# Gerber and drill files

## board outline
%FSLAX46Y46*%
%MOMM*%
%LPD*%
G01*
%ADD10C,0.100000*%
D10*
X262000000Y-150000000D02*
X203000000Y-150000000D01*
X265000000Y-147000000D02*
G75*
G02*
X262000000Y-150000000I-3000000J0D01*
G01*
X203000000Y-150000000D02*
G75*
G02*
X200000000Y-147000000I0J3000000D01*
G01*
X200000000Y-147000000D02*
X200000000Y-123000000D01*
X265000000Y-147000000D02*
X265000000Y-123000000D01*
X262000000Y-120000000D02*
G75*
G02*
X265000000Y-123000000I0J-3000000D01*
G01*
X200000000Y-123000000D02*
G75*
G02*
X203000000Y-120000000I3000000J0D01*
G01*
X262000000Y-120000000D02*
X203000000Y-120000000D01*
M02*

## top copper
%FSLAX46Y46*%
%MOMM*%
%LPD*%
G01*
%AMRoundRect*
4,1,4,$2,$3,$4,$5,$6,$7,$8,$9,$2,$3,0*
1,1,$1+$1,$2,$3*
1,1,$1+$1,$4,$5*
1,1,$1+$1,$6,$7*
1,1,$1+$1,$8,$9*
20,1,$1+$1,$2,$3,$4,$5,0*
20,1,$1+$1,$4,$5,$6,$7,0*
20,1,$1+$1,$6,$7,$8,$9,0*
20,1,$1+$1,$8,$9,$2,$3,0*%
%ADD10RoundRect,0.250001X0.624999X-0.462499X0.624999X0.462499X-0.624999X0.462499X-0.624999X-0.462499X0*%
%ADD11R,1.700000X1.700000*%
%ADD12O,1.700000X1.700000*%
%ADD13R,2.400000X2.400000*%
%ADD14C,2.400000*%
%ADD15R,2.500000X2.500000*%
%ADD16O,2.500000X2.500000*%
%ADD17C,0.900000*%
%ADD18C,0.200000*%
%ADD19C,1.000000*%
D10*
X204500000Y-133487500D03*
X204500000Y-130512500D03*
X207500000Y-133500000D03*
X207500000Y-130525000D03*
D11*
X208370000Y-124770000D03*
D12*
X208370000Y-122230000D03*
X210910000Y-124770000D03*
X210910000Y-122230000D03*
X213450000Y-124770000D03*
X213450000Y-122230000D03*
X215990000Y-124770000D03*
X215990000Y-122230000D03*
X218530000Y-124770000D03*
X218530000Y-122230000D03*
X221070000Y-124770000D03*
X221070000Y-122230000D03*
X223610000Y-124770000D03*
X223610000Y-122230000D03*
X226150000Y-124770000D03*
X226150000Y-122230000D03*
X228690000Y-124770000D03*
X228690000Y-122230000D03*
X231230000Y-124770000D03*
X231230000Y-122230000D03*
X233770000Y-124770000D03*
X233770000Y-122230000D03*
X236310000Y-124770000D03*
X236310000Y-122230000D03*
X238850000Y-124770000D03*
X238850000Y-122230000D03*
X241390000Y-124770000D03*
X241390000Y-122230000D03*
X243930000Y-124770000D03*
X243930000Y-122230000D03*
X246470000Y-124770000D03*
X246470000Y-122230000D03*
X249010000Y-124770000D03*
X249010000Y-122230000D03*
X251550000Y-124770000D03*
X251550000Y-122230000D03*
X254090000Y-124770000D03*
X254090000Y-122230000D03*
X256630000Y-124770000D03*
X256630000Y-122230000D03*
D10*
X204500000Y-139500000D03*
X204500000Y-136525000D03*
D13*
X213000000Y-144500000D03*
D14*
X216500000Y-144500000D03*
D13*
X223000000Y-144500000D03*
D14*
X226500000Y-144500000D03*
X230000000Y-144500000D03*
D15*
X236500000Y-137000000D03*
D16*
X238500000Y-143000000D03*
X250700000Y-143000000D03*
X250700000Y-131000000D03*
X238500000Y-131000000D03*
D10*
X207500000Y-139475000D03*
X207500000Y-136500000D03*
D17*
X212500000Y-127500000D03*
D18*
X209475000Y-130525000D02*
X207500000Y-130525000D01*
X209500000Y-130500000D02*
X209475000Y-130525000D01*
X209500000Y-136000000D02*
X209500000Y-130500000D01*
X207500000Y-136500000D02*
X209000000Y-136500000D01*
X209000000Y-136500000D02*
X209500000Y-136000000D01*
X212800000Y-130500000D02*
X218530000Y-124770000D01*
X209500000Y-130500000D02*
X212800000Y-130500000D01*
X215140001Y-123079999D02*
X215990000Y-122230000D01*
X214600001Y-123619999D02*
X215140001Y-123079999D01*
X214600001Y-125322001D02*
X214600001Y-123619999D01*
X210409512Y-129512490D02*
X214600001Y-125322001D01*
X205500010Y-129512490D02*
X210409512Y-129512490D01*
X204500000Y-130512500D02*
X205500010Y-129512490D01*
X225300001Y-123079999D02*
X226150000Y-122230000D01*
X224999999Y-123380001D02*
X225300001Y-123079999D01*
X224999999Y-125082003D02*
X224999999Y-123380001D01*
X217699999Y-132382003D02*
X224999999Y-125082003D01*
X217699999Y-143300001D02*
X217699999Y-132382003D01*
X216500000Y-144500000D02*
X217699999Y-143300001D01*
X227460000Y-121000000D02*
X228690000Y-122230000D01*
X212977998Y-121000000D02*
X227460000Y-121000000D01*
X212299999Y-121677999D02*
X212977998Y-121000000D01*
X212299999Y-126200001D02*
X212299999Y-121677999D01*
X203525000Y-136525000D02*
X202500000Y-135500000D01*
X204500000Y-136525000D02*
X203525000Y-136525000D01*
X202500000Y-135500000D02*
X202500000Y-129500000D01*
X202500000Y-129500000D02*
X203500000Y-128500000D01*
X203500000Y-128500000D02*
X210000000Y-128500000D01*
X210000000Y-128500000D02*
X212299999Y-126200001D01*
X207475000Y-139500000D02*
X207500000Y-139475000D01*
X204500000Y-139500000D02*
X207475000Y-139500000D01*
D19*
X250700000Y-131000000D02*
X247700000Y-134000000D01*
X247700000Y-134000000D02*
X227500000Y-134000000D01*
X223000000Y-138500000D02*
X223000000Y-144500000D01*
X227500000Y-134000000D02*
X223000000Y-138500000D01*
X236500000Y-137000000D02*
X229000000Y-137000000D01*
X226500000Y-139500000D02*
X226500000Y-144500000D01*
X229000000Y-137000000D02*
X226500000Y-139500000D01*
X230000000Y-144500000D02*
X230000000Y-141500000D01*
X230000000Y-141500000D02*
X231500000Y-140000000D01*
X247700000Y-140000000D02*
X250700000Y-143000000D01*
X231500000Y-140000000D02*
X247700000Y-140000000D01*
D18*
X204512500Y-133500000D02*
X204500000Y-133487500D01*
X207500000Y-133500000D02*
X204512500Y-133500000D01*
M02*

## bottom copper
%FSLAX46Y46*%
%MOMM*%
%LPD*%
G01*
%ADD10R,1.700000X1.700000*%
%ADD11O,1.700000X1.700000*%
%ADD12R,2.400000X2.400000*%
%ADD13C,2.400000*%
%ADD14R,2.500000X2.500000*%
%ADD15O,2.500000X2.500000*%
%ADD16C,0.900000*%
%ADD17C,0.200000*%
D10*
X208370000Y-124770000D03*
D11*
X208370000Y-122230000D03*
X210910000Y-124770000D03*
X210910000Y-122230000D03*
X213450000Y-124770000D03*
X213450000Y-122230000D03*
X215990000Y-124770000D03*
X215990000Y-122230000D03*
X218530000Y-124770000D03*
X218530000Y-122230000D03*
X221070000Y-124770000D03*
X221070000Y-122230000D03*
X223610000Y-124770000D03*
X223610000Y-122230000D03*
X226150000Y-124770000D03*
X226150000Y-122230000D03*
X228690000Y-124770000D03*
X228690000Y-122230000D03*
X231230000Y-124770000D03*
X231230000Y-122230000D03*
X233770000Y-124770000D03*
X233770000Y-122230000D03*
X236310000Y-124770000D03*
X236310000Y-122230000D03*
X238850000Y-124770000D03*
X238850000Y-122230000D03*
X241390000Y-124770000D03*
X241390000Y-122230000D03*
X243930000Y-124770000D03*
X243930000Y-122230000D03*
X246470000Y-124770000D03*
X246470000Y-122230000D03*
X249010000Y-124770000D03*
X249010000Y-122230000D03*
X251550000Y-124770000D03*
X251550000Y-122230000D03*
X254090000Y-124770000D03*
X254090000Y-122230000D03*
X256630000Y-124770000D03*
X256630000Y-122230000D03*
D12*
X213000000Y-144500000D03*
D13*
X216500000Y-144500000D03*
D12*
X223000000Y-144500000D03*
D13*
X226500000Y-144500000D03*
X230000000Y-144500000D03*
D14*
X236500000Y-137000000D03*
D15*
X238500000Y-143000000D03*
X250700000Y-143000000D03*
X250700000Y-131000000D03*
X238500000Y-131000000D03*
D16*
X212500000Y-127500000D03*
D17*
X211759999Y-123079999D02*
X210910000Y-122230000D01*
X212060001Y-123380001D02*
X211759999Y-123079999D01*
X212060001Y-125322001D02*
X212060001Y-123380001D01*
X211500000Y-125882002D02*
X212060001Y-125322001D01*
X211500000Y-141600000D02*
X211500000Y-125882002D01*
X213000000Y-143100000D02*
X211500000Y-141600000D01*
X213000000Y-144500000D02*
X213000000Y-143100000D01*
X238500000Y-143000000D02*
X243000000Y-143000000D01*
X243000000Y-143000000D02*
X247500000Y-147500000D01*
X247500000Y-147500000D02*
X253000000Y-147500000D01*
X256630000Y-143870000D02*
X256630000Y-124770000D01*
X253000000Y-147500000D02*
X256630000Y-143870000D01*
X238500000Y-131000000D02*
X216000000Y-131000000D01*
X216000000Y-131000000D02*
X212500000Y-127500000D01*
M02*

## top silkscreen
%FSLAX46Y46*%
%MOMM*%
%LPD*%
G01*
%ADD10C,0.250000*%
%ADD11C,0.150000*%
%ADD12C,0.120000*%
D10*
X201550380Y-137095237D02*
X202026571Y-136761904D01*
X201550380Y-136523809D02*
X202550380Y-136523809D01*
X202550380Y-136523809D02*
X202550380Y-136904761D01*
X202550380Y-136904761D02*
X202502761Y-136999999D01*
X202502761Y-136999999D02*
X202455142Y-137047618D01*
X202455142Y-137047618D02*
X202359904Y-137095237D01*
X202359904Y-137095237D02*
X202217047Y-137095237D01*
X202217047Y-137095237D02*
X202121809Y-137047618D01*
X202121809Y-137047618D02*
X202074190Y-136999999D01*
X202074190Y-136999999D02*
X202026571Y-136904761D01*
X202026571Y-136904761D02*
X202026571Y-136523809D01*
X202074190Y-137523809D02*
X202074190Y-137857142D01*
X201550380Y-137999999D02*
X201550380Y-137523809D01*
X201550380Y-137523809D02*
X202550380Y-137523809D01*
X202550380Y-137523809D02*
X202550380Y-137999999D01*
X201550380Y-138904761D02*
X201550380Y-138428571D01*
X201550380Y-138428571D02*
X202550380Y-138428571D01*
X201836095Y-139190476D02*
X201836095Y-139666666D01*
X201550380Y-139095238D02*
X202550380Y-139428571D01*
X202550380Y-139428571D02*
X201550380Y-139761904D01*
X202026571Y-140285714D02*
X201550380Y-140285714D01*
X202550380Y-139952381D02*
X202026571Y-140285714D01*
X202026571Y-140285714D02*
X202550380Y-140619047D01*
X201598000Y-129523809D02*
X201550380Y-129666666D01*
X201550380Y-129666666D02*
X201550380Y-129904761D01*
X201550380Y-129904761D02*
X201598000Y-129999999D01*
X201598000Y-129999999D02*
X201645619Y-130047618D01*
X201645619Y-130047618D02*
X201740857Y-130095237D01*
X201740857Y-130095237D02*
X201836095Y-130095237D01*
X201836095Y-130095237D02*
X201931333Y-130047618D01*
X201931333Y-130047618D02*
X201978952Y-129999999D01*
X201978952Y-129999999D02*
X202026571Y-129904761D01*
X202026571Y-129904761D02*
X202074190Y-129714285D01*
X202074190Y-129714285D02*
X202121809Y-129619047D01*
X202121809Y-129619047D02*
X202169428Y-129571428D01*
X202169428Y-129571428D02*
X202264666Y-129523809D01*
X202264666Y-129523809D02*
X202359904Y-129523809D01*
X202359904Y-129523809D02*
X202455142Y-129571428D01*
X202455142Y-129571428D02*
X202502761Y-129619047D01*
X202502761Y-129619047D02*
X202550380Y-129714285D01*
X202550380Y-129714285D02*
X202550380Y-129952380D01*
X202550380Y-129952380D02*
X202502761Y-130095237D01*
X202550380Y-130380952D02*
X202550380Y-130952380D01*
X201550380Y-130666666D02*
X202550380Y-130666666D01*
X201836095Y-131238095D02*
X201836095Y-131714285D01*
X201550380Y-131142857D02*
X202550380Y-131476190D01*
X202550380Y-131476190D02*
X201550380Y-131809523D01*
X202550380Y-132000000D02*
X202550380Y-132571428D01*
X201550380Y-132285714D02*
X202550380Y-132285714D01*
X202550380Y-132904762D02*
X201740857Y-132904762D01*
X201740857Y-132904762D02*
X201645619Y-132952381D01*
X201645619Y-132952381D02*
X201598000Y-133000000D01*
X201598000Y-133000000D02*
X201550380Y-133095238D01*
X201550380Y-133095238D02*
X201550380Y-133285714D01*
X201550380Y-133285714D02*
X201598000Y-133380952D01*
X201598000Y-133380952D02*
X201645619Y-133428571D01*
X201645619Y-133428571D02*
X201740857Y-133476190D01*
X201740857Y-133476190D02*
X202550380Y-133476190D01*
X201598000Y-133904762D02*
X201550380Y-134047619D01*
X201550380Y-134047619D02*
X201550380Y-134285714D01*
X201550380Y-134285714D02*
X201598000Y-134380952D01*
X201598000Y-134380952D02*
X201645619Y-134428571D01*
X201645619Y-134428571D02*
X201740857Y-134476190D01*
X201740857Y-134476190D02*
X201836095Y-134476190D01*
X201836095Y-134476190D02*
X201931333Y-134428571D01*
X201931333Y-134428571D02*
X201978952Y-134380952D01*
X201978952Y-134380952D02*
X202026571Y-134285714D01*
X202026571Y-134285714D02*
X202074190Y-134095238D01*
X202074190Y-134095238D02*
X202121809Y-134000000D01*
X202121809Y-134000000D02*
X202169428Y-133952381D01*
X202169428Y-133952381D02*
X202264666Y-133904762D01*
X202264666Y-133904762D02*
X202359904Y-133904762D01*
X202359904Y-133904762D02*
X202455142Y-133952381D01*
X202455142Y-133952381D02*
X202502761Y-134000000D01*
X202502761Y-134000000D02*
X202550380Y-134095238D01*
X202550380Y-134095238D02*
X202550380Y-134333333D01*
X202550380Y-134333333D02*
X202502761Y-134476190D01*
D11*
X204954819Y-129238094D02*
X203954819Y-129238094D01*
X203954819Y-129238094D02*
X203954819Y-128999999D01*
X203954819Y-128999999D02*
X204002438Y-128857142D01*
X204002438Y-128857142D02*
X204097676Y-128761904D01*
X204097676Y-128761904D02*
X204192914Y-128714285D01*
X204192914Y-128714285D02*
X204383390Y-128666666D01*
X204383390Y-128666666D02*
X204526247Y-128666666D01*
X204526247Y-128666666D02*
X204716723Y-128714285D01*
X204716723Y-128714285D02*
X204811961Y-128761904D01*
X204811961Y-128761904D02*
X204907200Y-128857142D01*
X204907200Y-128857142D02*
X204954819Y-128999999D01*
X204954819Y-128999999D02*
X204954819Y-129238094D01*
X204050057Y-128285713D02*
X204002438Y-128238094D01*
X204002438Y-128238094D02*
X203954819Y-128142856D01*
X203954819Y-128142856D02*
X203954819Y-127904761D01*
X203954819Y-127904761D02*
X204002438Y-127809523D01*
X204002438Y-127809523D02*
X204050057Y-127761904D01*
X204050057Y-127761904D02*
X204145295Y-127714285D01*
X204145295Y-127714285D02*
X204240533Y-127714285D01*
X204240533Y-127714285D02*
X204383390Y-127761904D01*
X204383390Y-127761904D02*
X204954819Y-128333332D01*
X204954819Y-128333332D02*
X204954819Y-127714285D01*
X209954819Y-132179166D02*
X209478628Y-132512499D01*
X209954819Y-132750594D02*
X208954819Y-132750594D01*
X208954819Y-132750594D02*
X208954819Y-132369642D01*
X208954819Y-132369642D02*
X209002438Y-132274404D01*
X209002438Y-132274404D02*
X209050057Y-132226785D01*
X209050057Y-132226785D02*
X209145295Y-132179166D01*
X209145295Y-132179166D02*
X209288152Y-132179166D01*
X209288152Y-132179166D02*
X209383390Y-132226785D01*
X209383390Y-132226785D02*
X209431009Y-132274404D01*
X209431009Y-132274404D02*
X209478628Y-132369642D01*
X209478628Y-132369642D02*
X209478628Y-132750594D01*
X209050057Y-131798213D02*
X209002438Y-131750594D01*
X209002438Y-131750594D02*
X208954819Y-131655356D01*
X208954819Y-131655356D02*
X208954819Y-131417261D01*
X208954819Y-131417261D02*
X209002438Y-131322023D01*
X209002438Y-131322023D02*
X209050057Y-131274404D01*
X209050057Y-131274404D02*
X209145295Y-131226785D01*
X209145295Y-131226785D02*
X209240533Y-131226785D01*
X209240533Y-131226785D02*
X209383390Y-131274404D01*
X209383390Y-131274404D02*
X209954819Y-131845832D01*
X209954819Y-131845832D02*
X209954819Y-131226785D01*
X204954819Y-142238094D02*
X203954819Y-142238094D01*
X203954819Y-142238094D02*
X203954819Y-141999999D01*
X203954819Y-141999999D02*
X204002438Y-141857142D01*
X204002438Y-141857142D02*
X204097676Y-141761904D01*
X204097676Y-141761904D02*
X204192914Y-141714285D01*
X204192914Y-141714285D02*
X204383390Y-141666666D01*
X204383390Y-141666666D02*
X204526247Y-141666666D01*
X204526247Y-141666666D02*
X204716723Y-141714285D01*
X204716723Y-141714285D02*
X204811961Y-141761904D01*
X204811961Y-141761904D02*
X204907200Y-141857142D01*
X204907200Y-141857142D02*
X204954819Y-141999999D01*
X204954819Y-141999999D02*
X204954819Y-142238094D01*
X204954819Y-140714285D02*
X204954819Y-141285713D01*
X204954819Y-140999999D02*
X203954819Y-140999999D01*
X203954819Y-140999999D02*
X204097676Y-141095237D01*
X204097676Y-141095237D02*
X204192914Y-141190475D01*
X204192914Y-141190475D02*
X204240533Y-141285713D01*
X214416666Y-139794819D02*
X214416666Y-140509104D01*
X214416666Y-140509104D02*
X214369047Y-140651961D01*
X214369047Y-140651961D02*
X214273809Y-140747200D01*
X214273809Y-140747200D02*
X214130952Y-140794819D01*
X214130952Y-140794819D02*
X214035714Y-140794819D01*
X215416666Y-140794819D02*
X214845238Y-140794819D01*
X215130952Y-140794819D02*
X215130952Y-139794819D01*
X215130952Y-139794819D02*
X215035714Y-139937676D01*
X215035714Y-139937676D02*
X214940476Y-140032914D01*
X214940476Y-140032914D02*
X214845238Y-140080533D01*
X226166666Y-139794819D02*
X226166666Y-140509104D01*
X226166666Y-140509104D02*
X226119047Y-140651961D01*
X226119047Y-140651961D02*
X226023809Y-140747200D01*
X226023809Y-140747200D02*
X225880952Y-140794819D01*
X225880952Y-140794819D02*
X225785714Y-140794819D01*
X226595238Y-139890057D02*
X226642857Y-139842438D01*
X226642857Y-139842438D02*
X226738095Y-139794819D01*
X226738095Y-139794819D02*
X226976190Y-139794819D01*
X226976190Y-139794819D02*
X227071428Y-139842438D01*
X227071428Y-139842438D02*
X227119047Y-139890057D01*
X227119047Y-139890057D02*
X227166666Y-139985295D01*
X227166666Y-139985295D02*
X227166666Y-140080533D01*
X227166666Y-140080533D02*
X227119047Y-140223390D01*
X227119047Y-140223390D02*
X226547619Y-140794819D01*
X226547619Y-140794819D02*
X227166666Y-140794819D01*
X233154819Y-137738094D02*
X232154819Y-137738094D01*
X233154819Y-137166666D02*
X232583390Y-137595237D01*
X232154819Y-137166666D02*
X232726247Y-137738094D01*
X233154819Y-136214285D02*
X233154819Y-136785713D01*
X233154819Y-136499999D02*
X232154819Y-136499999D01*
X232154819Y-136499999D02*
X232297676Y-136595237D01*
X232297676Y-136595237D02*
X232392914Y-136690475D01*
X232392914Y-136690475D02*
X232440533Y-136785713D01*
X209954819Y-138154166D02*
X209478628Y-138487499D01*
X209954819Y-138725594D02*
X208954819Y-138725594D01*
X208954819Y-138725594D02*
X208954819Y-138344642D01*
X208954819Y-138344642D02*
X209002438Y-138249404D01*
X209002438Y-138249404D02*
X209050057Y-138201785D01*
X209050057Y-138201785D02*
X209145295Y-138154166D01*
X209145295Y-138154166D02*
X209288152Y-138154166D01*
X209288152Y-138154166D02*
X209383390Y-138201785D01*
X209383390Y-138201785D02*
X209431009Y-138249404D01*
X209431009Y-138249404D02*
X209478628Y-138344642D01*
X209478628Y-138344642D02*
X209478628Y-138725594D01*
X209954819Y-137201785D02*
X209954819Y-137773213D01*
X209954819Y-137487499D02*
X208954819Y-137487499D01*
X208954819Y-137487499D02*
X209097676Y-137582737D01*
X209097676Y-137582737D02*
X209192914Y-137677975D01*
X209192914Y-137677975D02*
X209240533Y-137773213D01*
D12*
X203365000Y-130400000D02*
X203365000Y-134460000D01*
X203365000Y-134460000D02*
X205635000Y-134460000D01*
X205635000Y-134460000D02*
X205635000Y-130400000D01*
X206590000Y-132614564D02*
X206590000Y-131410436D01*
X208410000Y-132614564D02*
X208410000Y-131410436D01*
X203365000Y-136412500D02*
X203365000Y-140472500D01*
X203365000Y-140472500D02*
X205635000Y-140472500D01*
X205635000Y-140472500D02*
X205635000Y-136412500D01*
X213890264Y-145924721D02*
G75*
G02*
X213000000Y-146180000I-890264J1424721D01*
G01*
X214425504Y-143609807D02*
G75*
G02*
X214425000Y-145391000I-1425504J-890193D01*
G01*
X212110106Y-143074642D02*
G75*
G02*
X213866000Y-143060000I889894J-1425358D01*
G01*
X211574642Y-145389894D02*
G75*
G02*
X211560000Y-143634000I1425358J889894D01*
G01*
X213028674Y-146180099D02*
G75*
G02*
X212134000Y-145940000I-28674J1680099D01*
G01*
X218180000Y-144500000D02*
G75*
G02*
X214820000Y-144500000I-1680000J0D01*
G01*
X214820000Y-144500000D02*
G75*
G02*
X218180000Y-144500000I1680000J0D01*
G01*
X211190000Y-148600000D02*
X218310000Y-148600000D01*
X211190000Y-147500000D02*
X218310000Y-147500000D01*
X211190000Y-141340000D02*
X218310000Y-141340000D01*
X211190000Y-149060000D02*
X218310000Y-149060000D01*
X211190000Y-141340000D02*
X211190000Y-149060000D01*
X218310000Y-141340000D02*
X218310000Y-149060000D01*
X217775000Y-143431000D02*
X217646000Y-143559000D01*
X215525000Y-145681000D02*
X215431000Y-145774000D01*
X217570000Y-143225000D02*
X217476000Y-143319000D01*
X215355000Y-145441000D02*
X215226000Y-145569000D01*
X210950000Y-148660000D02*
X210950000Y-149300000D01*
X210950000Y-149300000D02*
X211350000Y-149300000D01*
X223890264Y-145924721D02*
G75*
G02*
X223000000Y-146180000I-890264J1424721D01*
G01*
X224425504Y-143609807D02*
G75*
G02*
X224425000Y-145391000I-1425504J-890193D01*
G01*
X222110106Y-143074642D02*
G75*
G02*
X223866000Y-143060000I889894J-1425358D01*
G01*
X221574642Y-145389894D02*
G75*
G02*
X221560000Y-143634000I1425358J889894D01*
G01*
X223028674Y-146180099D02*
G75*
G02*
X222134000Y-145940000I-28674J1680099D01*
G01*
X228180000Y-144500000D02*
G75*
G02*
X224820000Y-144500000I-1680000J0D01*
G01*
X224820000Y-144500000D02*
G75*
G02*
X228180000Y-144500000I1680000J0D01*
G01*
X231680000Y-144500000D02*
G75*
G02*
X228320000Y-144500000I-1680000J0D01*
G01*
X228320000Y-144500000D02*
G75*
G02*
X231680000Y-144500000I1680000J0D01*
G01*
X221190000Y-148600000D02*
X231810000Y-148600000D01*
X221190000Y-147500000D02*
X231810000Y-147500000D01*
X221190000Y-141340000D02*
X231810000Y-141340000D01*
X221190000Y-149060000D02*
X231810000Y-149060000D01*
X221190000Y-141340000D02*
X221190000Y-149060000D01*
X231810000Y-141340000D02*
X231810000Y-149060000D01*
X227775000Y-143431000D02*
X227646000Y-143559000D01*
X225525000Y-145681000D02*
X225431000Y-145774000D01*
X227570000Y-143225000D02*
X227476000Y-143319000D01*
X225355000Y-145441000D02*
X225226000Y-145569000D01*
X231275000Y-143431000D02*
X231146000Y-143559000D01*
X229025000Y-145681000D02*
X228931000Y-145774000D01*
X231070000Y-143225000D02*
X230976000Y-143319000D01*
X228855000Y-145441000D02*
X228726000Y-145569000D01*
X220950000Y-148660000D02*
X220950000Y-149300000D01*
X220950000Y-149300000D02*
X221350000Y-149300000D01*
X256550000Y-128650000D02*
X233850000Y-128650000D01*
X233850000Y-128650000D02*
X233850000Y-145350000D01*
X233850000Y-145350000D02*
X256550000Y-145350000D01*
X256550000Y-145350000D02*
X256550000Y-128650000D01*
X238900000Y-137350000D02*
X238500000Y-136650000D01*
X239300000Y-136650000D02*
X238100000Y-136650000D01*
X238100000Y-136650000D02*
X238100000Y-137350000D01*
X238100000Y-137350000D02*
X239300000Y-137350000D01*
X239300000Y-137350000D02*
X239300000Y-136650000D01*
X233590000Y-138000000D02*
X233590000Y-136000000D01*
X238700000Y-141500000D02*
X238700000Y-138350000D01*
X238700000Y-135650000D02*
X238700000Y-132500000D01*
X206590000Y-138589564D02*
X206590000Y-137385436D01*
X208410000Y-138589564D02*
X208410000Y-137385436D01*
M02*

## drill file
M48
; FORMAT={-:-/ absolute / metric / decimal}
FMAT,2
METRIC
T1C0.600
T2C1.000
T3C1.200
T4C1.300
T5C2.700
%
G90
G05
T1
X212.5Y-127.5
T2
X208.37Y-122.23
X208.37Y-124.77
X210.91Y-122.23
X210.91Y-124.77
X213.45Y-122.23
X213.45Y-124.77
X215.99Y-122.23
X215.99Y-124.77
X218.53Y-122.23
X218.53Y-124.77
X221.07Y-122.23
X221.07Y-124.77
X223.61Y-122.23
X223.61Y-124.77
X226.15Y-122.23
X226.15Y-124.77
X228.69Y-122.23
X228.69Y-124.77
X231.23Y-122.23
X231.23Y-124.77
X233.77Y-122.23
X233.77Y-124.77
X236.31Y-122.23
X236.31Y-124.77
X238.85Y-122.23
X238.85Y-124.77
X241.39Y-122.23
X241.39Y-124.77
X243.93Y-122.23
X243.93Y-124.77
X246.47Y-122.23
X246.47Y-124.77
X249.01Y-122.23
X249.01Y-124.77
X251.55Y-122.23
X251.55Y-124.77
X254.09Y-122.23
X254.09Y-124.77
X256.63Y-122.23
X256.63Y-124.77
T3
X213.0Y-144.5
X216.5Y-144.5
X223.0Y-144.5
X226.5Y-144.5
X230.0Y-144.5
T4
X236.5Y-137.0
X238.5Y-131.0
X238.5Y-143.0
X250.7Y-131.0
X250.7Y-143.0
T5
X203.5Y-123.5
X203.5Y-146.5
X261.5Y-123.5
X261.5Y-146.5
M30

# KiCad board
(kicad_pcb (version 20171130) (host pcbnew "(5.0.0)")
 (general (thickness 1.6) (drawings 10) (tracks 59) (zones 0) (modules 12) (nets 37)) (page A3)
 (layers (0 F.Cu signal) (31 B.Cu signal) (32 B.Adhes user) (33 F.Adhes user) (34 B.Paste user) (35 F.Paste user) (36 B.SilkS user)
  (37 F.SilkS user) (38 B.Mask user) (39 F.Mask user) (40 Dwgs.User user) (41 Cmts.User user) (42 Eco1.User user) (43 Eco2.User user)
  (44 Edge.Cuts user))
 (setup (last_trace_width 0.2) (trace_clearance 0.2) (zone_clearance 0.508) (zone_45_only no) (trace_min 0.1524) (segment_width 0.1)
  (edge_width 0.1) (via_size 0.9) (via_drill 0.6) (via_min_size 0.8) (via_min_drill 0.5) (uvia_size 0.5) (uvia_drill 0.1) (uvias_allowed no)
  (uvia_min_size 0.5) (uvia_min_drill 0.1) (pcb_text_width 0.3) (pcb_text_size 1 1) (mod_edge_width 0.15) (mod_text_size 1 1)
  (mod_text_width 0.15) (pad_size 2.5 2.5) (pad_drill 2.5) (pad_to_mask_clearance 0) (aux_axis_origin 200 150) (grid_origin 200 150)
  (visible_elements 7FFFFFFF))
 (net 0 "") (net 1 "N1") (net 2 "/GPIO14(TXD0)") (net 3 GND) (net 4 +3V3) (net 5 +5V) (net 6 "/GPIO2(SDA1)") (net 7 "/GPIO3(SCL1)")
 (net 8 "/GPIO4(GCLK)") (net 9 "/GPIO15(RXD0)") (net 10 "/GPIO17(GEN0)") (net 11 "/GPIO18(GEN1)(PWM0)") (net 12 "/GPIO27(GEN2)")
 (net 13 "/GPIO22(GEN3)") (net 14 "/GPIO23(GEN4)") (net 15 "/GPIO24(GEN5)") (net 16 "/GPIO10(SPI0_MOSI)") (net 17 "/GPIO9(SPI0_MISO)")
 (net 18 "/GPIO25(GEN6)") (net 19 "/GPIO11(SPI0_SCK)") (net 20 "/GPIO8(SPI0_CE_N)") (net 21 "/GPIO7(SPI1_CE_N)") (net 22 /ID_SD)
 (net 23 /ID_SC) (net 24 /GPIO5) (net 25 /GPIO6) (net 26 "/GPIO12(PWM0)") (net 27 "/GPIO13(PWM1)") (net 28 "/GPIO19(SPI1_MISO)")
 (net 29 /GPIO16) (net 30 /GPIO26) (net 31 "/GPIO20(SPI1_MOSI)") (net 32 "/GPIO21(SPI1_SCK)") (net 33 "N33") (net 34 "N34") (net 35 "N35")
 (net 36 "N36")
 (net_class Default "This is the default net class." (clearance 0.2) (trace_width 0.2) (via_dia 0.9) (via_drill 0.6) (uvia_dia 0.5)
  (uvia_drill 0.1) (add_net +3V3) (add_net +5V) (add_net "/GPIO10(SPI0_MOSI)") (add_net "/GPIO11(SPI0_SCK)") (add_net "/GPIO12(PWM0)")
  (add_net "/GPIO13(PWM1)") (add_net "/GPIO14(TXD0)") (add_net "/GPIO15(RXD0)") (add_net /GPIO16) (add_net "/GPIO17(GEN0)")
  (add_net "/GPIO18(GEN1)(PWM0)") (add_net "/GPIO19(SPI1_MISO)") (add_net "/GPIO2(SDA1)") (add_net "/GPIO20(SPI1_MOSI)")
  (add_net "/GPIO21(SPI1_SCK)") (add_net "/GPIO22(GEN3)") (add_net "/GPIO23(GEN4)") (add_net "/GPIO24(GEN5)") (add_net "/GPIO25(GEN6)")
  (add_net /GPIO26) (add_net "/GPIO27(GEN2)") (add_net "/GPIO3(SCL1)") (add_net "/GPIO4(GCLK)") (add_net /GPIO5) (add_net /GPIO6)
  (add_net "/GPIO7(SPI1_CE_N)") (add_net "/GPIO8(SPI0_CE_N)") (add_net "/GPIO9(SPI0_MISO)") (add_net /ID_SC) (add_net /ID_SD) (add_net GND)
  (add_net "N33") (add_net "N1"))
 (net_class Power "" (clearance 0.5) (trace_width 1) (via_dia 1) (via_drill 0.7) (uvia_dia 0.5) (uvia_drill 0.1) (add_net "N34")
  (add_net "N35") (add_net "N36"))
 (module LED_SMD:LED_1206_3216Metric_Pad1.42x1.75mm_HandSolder (layer F.Cu) (at 204.5 132 90)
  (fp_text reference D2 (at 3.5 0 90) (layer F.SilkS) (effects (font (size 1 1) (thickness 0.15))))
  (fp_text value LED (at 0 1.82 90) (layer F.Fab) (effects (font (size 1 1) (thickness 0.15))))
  (fp_line (start 1.6 -1.135) (end -2.46 -1.135) (layer F.SilkS) (width 0.12))
  (fp_line (start -2.46 -1.135) (end -2.46 1.135) (layer F.SilkS) (width 0.12))
  (fp_line (start -2.46 1.135) (end 1.6 1.135) (layer F.SilkS) (width 0.12))
  (pad 1 smd roundrect (at -1.4875 0 90) (size 1.425 1.75) (layers F.Cu F.Paste F.Mask) (roundrect_rratio 0.175439) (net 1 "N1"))
  (pad 2 smd roundrect (at 1.4875 0 90) (size 1.425 1.75) (layers F.Cu F.Paste F.Mask) (roundrect_rratio 0.175439) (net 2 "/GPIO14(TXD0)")))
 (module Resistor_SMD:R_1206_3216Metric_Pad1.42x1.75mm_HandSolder (layer F.Cu) (at 207.5 132.0125 90)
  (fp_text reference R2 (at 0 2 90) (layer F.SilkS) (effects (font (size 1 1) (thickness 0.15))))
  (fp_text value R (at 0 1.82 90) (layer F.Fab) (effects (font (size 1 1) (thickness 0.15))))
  (fp_line (start -0.602064 -0.91) (end 0.602064 -0.91) (layer F.SilkS) (width 0.12))
  (fp_line (start -0.602064 0.91) (end 0.602064 0.91) (layer F.SilkS) (width 0.12))
  (pad 1 smd roundrect (at -1.4875 0 90) (size 1.425 1.75) (layers F.Cu F.Paste F.Mask) (roundrect_rratio 0.175439) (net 1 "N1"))
  (pad 2 smd roundrect (at 1.4875 0 90) (size 1.425 1.75) (layers F.Cu F.Paste F.Mask) (roundrect_rratio 0.175439) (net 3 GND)))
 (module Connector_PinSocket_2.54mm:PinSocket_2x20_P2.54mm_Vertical (layer B.Cu) (at 208.37 124.77 270)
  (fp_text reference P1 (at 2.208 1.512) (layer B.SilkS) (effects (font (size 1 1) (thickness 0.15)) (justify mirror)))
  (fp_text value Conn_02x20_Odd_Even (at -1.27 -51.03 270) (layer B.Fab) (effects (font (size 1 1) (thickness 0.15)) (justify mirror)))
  (pad 1 thru_hole rect (at 0 0 270) (size 1.7 1.7) (drill 1) (layers *.Cu *.Mask) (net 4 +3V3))
  (pad 2 thru_hole oval (at -2.54 0 270) (size 1.7 1.7) (drill 1) (layers *.Cu *.Mask) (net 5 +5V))
  (pad 3 thru_hole oval (at 0 -2.54 270) (size 1.7 1.7) (drill 1) (layers *.Cu *.Mask) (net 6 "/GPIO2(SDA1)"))
  (pad 4 thru_hole oval (at -2.54 -2.54 270) (size 1.7 1.7) (drill 1) (layers *.Cu *.Mask) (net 5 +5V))
  (pad 5 thru_hole oval (at 0 -5.08 270) (size 1.7 1.7) (drill 1) (layers *.Cu *.Mask) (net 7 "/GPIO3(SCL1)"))
  (pad 6 thru_hole oval (at -2.54 -5.08 270) (size 1.7 1.7) (drill 1) (layers *.Cu *.Mask) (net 3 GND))
  (pad 7 thru_hole oval (at 0 -7.62 270) (size 1.7 1.7) (drill 1) (layers *.Cu *.Mask) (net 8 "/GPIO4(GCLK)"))
  (pad 8 thru_hole oval (at -2.54 -7.62 270) (size 1.7 1.7) (drill 1) (layers *.Cu *.Mask) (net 2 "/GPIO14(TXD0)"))
  (pad 9 thru_hole oval (at 0 -10.16 270) (size 1.7 1.7) (drill 1) (layers *.Cu *.Mask) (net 3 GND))
  (pad 10 thru_hole oval (at -2.54 -10.16 270) (size 1.7 1.7) (drill 1) (layers *.Cu *.Mask) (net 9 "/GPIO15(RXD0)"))
  (pad 11 thru_hole oval (at 0 -12.7 270) (size 1.7 1.7) (drill 1) (layers *.Cu *.Mask) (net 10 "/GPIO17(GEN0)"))
  (pad 12 thru_hole oval (at -2.54 -12.7 270) (size 1.7 1.7) (drill 1) (layers *.Cu *.Mask) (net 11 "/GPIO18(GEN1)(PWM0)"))
  (pad 13 thru_hole oval (at 0 -15.24 270) (size 1.7 1.7) (drill 1) (layers *.Cu *.Mask) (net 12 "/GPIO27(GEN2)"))
  (pad 14 thru_hole oval (at -2.54 -15.24 270) (size 1.7 1.7) (drill 1) (layers *.Cu *.Mask) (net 3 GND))
  (pad 15 thru_hole oval (at 0 -17.78 270) (size 1.7 1.7) (drill 1) (layers *.Cu *.Mask) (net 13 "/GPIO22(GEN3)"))
  (pad 16 thru_hole oval (at -2.54 -17.78 270) (size 1.7 1.7) (drill 1) (layers *.Cu *.Mask) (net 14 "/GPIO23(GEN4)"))
  (pad 17 thru_hole oval (at 0 -20.32 270) (size 1.7 1.7) (drill 1) (layers *.Cu *.Mask) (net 4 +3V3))
  (pad 18 thru_hole oval (at -2.54 -20.32 270) (size 1.7 1.7) (drill 1) (layers *.Cu *.Mask) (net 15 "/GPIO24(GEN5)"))
  (pad 19 thru_hole oval (at 0 -22.86 270) (size 1.7 1.7) (drill 1) (layers *.Cu *.Mask) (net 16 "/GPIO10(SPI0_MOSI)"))
  (pad 20 thru_hole oval (at -2.54 -22.86 270) (size 1.7 1.7) (drill 1) (layers *.Cu *.Mask) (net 3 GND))
  (pad 21 thru_hole oval (at 0 -25.4 270) (size 1.7 1.7) (drill 1) (layers *.Cu *.Mask) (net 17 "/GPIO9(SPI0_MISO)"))
  (pad 22 thru_hole oval (at -2.54 -25.4 270) (size 1.7 1.7) (drill 1) (layers *.Cu *.Mask) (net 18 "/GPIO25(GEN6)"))
  (pad 23 thru_hole oval (at 0 -27.94 270) (size 1.7 1.7) (drill 1) (layers *.Cu *.Mask) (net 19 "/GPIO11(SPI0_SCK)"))
  (pad 24 thru_hole oval (at -2.54 -27.94 270) (size 1.7 1.7) (drill 1) (layers *.Cu *.Mask) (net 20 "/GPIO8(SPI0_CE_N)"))
  (pad 25 thru_hole oval (at 0 -30.48 270) (size 1.7 1.7) (drill 1) (layers *.Cu *.Mask) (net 3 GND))
  (pad 26 thru_hole oval (at -2.54 -30.48 270) (size 1.7 1.7) (drill 1) (layers *.Cu *.Mask) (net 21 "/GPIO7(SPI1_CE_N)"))
  (pad 27 thru_hole oval (at 0 -33.02 270) (size 1.7 1.7) (drill 1) (layers *.Cu *.Mask) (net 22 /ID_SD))
  (pad 28 thru_hole oval (at -2.54 -33.02 270) (size 1.7 1.7) (drill 1) (layers *.Cu *.Mask) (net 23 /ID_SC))
  (pad 29 thru_hole oval (at 0 -35.56 270) (size 1.7 1.7) (drill 1) (layers *.Cu *.Mask) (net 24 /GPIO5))
  (pad 30 thru_hole oval (at -2.54 -35.56 270) (size 1.7 1.7) (drill 1) (layers *.Cu *.Mask) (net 3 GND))
  (pad 31 thru_hole oval (at 0 -38.1 270) (size 1.7 1.7) (drill 1) (layers *.Cu *.Mask) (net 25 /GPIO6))
  (pad 32 thru_hole oval (at -2.54 -38.1 270) (size 1.7 1.7) (drill 1) (layers *.Cu *.Mask) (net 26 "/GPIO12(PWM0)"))
  (pad 33 thru_hole oval (at 0 -40.64 270) (size 1.7 1.7) (drill 1) (layers *.Cu *.Mask) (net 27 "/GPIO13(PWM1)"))
  (pad 34 thru_hole oval (at -2.54 -40.64 270) (size 1.7 1.7) (drill 1) (layers *.Cu *.Mask) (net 3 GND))
  (pad 35 thru_hole oval (at 0 -43.18 270) (size 1.7 1.7) (drill 1) (layers *.Cu *.Mask) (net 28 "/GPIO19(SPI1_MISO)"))
  (pad 36 thru_hole oval (at -2.54 -43.18 270) (size 1.7 1.7) (drill 1) (layers *.Cu *.Mask) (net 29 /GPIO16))
  (pad 37 thru_hole oval (at 0 -45.72 270) (size 1.7 1.7) (drill 1) (layers *.Cu *.Mask) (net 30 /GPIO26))
  (pad 38 thru_hole oval (at -2.54 -45.72 270) (size 1.7 1.7) (drill 1) (layers *.Cu *.Mask) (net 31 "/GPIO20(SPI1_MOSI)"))
  (pad 39 thru_hole oval (at 0 -48.26 270) (size 1.7 1.7) (drill 1) (layers *.Cu *.Mask) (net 3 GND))
  (pad 40 thru_hole oval (at -2.54 -48.26 270) (size 1.7 1.7) (drill 1) (layers *.Cu *.Mask) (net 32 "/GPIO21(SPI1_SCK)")))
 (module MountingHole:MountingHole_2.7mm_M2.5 (layer F.Cu) (at 261.5 146.5)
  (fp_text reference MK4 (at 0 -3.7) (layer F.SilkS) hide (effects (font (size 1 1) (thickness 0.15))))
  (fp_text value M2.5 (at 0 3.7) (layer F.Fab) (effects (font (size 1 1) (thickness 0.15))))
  (pad 1 np_thru_hole circle (at 0 0) (size 2.7 2.7) (drill 2.7) (layers *.Cu *.Mask)))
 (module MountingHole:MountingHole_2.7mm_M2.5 (layer F.Cu) (at 203.5 146.5)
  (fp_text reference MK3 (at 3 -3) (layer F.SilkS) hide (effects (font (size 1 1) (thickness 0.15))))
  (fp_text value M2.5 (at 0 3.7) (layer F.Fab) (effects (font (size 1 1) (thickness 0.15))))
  (pad 1 np_thru_hole circle (at 0 0) (size 2.7 2.7) (drill 2.7) (layers *.Cu *.Mask)))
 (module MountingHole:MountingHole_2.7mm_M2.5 (layer F.Cu) (at 261.5 123.5 180)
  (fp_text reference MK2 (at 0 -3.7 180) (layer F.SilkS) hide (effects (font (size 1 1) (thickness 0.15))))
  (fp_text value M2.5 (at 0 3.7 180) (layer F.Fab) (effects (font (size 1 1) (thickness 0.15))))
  (pad 1 np_thru_hole circle (at 0 0 180) (size 2.7 2.7) (drill 2.7) (layers *.Cu *.Mask)))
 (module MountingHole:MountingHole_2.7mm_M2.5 (layer F.Cu) (at 203.5 123.5 180)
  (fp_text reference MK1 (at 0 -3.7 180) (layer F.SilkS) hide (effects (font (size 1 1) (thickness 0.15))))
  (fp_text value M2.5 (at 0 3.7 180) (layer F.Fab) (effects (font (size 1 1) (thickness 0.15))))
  (pad 1 np_thru_hole circle (at 0 0 180) (size 2.7 2.7) (drill 2.7) (layers *.Cu *.Mask)))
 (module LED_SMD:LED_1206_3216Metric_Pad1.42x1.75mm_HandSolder (layer F.Cu) (at 204.5 138.0125 90)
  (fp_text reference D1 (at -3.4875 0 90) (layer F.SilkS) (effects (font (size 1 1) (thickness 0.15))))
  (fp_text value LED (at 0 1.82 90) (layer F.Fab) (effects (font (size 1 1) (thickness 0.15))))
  (fp_line (start 1.6 -1.135) (end -2.46 -1.135) (layer F.SilkS) (width 0.12))
  (fp_line (start -2.46 -1.135) (end -2.46 1.135) (layer F.SilkS) (width 0.12))
  (fp_line (start -2.46 1.135) (end 1.6 1.135) (layer F.SilkS) (width 0.12))
  (pad 1 smd roundrect (at -1.4875 0 90) (size 1.425 1.75) (layers F.Cu F.Paste F.Mask) (roundrect_rratio 0.175439) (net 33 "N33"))
  (pad 2 smd roundrect (at 1.4875 0 90) (size 1.425 1.75) (layers F.Cu F.Paste F.Mask) (roundrect_rratio 0.175439) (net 15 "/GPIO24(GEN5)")))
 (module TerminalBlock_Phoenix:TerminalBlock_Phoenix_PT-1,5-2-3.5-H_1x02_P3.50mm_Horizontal (layer F.Cu) (at 213 144.5)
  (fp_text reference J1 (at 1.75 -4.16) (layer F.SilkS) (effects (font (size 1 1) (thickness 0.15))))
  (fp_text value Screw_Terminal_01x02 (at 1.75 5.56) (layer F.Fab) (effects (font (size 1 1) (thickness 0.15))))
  (fp_arc (start 0 0) (end 0 1.68) (angle -32) (layer F.SilkS) (width 0.12))
  (fp_arc (start 0 0) (end 1.425 0.891) (angle -64) (layer F.SilkS) (width 0.12))
  (fp_arc (start 0 0) (end 0.866 -1.44) (angle -63) (layer F.SilkS) (width 0.12))
  (fp_arc (start 0 0) (end -1.44 -0.866) (angle -63) (layer F.SilkS) (width 0.12))
  (fp_arc (start 0 0) (end -0.866 1.44) (angle -32) (layer F.SilkS) (width 0.12))
  (fp_circle (center 3.5 0) (end 5.18 0) (layer F.SilkS) (width 0.12))
  (fp_line (start -1.81 4.1) (end 5.31 4.1) (layer F.SilkS) (width 0.12))
  (fp_line (start -1.81 3) (end 5.31 3) (layer F.SilkS) (width 0.12))
  (fp_line (start -1.81 -3.16) (end 5.31 -3.16) (layer F.SilkS) (width 0.12))
  (fp_line (start -1.81 4.56) (end 5.31 4.56) (layer F.SilkS) (width 0.12))
  (fp_line (start -1.81 -3.16) (end -1.81 4.56) (layer F.SilkS) (width 0.12))
  (fp_line (start 5.31 -3.16) (end 5.31 4.56) (layer F.SilkS) (width 0.12))
  (fp_line (start 4.775 -1.069) (end 4.646 -0.941) (layer F.SilkS) (width 0.12))
  (fp_line (start 2.525 1.181) (end 2.431 1.274) (layer F.SilkS) (width 0.12))
  (fp_line (start 4.57 -1.275) (end 4.476 -1.181) (layer F.SilkS) (width 0.12))
  (fp_line (start 2.355 0.941) (end 2.226 1.069) (layer F.SilkS) (width 0.12))
  (fp_line (start -2.05 4.16) (end -2.05 4.8) (layer F.SilkS) (width 0.12))
  (fp_line (start -2.05 4.8) (end -1.65 4.8) (layer F.SilkS) (width 0.12))
  (pad 1 thru_hole rect (at 0 0) (size 2.4 2.4) (drill 1.2) (layers *.Cu *.Mask) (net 5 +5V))
  (pad 2 thru_hole circle (at 3.5 0) (size 2.4 2.4) (drill 1.2) (layers *.Cu *.Mask) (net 14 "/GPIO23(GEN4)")))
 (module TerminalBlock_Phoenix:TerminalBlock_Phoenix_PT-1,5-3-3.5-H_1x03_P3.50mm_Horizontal (layer F.Cu) (at 223 144.5)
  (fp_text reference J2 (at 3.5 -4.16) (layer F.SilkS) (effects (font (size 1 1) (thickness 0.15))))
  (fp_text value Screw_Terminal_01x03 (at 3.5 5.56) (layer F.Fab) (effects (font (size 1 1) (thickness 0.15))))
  (fp_arc (start 0 0) (end 0 1.68) (angle -32) (layer F.SilkS) (width 0.12))
  (fp_arc (start 0 0) (end 1.425 0.891) (angle -64) (layer F.SilkS) (width 0.12))
  (fp_arc (start 0 0) (end 0.866 -1.44) (angle -63) (layer F.SilkS) (width 0.12))
  (fp_arc (start 0 0) (end -1.44 -0.866) (angle -63) (layer F.SilkS) (width 0.12))
  (fp_arc (start 0 0) (end -0.866 1.44) (angle -32) (layer F.SilkS) (width 0.12))
  (fp_circle (center 3.5 0) (end 5.18 0) (layer F.SilkS) (width 0.12))
  (fp_circle (center 7 0) (end 8.68 0) (layer F.SilkS) (width 0.12))
  (fp_line (start -1.81 4.1) (end 8.81 4.1) (layer F.SilkS) (width 0.12))
  (fp_line (start -1.81 3) (end 8.81 3) (layer F.SilkS) (width 0.12))
  (fp_line (start -1.81 -3.16) (end 8.81 -3.16) (layer F.SilkS) (width 0.12))
  (fp_line (start -1.81 4.56) (end 8.81 4.56) (layer F.SilkS) (width 0.12))
  (fp_line (start -1.81 -3.16) (end -1.81 4.56) (layer F.SilkS) (width 0.12))
  (fp_line (start 8.81 -3.16) (end 8.81 4.56) (layer F.SilkS) (width 0.12))
  (fp_line (start 4.775 -1.069) (end 4.646 -0.941) (layer F.SilkS) (width 0.12))
  (fp_line (start 2.525 1.181) (end 2.431 1.274) (layer F.SilkS) (width 0.12))
  (fp_line (start 4.57 -1.275) (end 4.476 -1.181) (layer F.SilkS) (width 0.12))
  (fp_line (start 2.355 0.941) (end 2.226 1.069) (layer F.SilkS) (width 0.12))
  (fp_line (start 8.275 -1.069) (end 8.146 -0.941) (layer F.SilkS) (width 0.12))
  (fp_line (start 6.025 1.181) (end 5.931 1.274) (layer F.SilkS) (width 0.12))
  (fp_line (start 8.07 -1.275) (end 7.976 -1.181) (layer F.SilkS) (width 0.12))
  (fp_line (start 5.855 0.941) (end 5.726 1.069) (layer F.SilkS) (width 0.12))
  (fp_line (start -2.05 4.16) (end -2.05 4.8) (layer F.SilkS) (width 0.12))
  (fp_line (start -2.05 4.8) (end -1.65 4.8) (layer F.SilkS) (width 0.12))
  (pad 1 thru_hole rect (at 0 0) (size 2.4 2.4) (drill 1.2) (layers *.Cu *.Mask) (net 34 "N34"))
  (pad 2 thru_hole circle (at 3.5 0) (size 2.4 2.4) (drill 1.2) (layers *.Cu *.Mask) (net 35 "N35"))
  (pad 3 thru_hole circle (at 7 0) (size 2.4 2.4) (drill 1.2) (layers *.Cu *.Mask) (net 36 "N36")))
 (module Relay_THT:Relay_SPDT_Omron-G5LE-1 (layer F.Cu) (at 236.5 137 90)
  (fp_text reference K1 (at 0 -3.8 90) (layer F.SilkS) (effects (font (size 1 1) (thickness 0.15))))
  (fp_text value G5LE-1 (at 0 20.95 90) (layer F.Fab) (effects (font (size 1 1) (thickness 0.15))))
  (fp_line (start 8.35 20.05) (end 8.35 -2.65) (layer F.SilkS) (width 0.12))
  (fp_line (start 8.35 -2.65) (end -8.35 -2.65) (layer F.SilkS) (width 0.12))
  (fp_line (start -8.35 -2.65) (end -8.35 20.05) (layer F.SilkS) (width 0.12))
  (fp_line (start -8.35 20.05) (end 8.35 20.05) (layer F.SilkS) (width 0.12))
  (fp_line (start -0.35 2.4) (end 0.35 2) (layer F.SilkS) (width 0.12))
  (fp_line (start 0.35 2.8) (end 0.35 1.6) (layer F.SilkS) (width 0.12))
  (fp_line (start 0.35 1.6) (end -0.35 1.6) (layer F.SilkS) (width 0.12))
  (fp_line (start -0.35 1.6) (end -0.35 2.8) (layer F.SilkS) (width 0.12))
  (fp_line (start -0.35 2.8) (end 0.35 2.8) (layer F.SilkS) (width 0.12))
  (fp_line (start -1 -2.91) (end 1 -2.91) (layer F.SilkS) (width 0.12))
  (fp_line (start -4.5 2.2) (end -1.35 2.2) (layer F.SilkS) (width 0.12))
  (fp_line (start 1.35 2.2) (end 4.5 2.2) (layer F.SilkS) (width 0.12))
  (pad 1 thru_hole rect (at 0 0 90) (size 2.5 2.5) (drill 1.3) (layers *.Cu *.Mask) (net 35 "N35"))
  (pad 2 thru_hole oval (at -6 2 90) (size 2.5 2.5) (drill 1.3) (layers *.Cu *.Mask) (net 3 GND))
  (pad 3 thru_hole oval (at -6 14.2 90) (size 2.5 2.5) (drill 1.3) (layers *.Cu *.Mask) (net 36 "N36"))
  (pad 4 thru_hole oval (at 6 14.2 90) (size 2.5 2.5) (drill 1.3) (layers *.Cu *.Mask) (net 34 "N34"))
  (pad 5 thru_hole oval (at 6 2 90) (size 2.5 2.5) (drill 1.3) (layers *.Cu *.Mask) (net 2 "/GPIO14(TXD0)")))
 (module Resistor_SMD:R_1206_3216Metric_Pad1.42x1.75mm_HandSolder (layer F.Cu) (at 207.5 137.9875 90)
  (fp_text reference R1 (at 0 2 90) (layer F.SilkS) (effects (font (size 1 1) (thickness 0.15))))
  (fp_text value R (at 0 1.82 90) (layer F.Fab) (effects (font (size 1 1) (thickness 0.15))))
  (fp_line (start -0.602064 -0.91) (end 0.602064 -0.91) (layer F.SilkS) (width 0.12))
  (fp_line (start -0.602064 0.91) (end 0.602064 0.91) (layer F.SilkS) (width 0.12))
  (pad 1 smd roundrect (at -1.4875 0 90) (size 1.425 1.75) (layers F.Cu F.Paste F.Mask) (roundrect_rratio 0.175439) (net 33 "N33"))
  (pad 2 smd roundrect (at 1.4875 0 90) (size 1.425 1.75) (layers F.Cu F.Paste F.Mask) (roundrect_rratio 0.175439) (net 3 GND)))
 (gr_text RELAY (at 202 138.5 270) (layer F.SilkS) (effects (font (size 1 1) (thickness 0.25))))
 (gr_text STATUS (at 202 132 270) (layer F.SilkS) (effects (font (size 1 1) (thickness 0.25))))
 (gr_line (start 262 150) (end 203 150) (layer Edge.Cuts) (width 0.1))
 (gr_arc (start 262 147) (end 262 150) (angle -90) (layer Edge.Cuts) (width 0.1))
 (gr_arc (start 203 147) (end 200 147) (angle -90) (layer Edge.Cuts) (width 0.1))
 (gr_line (start 200 147) (end 200 123) (layer Edge.Cuts) (width 0.1))
 (gr_line (start 265 147) (end 265 123) (layer Edge.Cuts) (width 0.1))
 (gr_arc (start 262 123) (end 262 120) (angle 90) (layer Edge.Cuts) (width 0.1))
 (gr_arc (start 203 123) (end 200 123) (angle 90) (layer Edge.Cuts) (width 0.1))
 (gr_line (start 262 120) (end 203 120) (layer Edge.Cuts) (width 0.1))
 (segment (start 211.759999 123.079999) (end 210.91 122.23) (width 0.2) (layer B.Cu) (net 5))
 (segment (start 212.060001 123.380001) (end 211.759999 123.079999) (width 0.2) (layer B.Cu) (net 5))
 (segment (start 212.060001 125.322001) (end 212.060001 123.380001) (width 0.2) (layer B.Cu) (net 5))
 (segment (start 211.5 125.882002) (end 212.060001 125.322001) (width 0.2) (layer B.Cu) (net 5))
 (segment (start 211.5 141.6) (end 211.5 125.882002) (width 0.2) (layer B.Cu) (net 5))
 (segment (start 213 143.1) (end 211.5 141.6) (width 0.2) (layer B.Cu) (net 5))
 (segment (start 213 144.5) (end 213 143.1) (width 0.2) (layer B.Cu) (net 5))
 (segment (start 209.475 130.525) (end 207.5 130.525) (width 0.2) (layer F.Cu) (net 3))
 (segment (start 209.5 130.5) (end 209.475 130.525) (width 0.2) (layer F.Cu) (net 3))
 (segment (start 209.5 136) (end 209.5 130.5) (width 0.2) (layer F.Cu) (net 3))
 (segment (start 207.5 136.5) (end 209 136.5) (width 0.2) (layer F.Cu) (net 3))
 (segment (start 209 136.5) (end 209.5 136) (width 0.2) (layer F.Cu) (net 3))
 (segment (start 212.8 130.5) (end 218.53 124.77) (width 0.2) (layer F.Cu) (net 3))
 (segment (start 209.5 130.5) (end 212.8 130.5) (width 0.2) (layer F.Cu) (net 3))
 (segment (start 238.5 143) (end 243 143) (width 0.2) (layer B.Cu) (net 3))
 (segment (start 243 143) (end 247.5 147.5) (width 0.2) (layer B.Cu) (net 3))
 (segment (start 247.5 147.5) (end 253 147.5) (width 0.2) (layer B.Cu) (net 3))
 (segment (start 256.63 143.87) (end 256.63 124.77) (width 0.2) (layer B.Cu) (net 3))
 (segment (start 253 147.5) (end 256.63 143.87) (width 0.2) (layer B.Cu) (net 3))
 (segment (start 215.140001 123.079999) (end 215.99 122.23) (width 0.2) (layer F.Cu) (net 2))
 (segment (start 214.600001 123.619999) (end 215.140001 123.079999) (width 0.2) (layer F.Cu) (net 2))
 (segment (start 214.600001 125.322001) (end 214.600001 123.619999) (width 0.2) (layer F.Cu) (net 2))
 (segment (start 210.409512 129.51249) (end 214.600001 125.322001) (width 0.2) (layer F.Cu) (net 2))
 (segment (start 205.50001 129.51249) (end 210.409512 129.51249) (width 0.2) (layer F.Cu) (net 2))
 (segment (start 204.5 130.5125) (end 205.50001 129.51249) (width 0.2) (layer F.Cu) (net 2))
 (segment (start 238.5 131) (end 216 131) (width 0.2) (layer B.Cu) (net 2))
 (via (at 212.5 127.5) (size 0.9) (drill 0.6) (layers F.Cu B.Cu) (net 2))
 (segment (start 216 131) (end 212.5 127.5) (width 0.2) (layer B.Cu) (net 2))
 (segment (start 225.300001 123.079999) (end 226.15 122.23) (width 0.2) (layer F.Cu) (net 14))
 (segment (start 224.999999 123.380001) (end 225.300001 123.079999) (width 0.2) (layer F.Cu) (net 14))
 (segment (start 224.999999 125.082003) (end 224.999999 123.380001) (width 0.2) (layer F.Cu) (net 14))
 (segment (start 217.699999 132.382003) (end 224.999999 125.082003) (width 0.2) (layer F.Cu) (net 14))
 (segment (start 217.699999 143.300001) (end 217.699999 132.382003) (width 0.2) (layer F.Cu) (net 14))
 (segment (start 216.5 144.5) (end 217.699999 143.300001) (width 0.2) (layer F.Cu) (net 14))
 (segment (start 227.46 121) (end 228.69 122.23) (width 0.2) (layer F.Cu) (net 15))
 (segment (start 212.977998 121) (end 227.46 121) (width 0.2) (layer F.Cu) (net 15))
 (segment (start 212.299999 121.677999) (end 212.977998 121) (width 0.2) (layer F.Cu) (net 15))
 (segment (start 212.299999 126.200001) (end 212.299999 121.677999) (width 0.2) (layer F.Cu) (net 15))
 (segment (start 203.525 136.525) (end 202.5 135.5) (width 0.2) (layer F.Cu) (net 15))
 (segment (start 204.5 136.525) (end 203.525 136.525) (width 0.2) (layer F.Cu) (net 15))
 (segment (start 202.5 135.5) (end 202.5 129.5) (width 0.2) (layer F.Cu) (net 15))
 (segment (start 202.5 129.5) (end 203.5 128.5) (width 0.2) (layer F.Cu) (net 15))
 (segment (start 203.5 128.5) (end 210 128.5) (width 0.2) (layer F.Cu) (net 15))
 (segment (start 210 128.5) (end 212.299999 126.200001) (width 0.2) (layer F.Cu) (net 15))
 (segment (start 207.475 139.5) (end 207.5 139.475) (width 0.2) (layer F.Cu) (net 33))
 (segment (start 204.5 139.5) (end 207.475 139.5) (width 0.2) (layer F.Cu) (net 33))
 (segment (start 250.7 131) (end 247.7 134) (width 1) (layer F.Cu) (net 34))
 (segment (start 247.7 134) (end 227.5 134) (width 1) (layer F.Cu) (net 34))
 (segment (start 223 138.5) (end 223 144.5) (width 1) (layer F.Cu) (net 34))
 (segment (start 227.5 134) (end 223 138.5) (width 1) (layer F.Cu) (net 34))
 (segment (start 236.5 137) (end 229 137) (width 1) (layer F.Cu) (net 35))
 (segment (start 226.5 139.5) (end 226.5 144.5) (width 1) (layer F.Cu) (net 35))
 (segment (start 229 137) (end 226.5 139.5) (width 1) (layer F.Cu) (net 35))
 (segment (start 230 144.5) (end 230 141.5) (width 1) (layer F.Cu) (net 36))
 (segment (start 230 141.5) (end 231.5 140) (width 1) (layer F.Cu) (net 36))
 (segment (start 247.7 140) (end 250.7 143) (width 1) (layer F.Cu) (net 36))
 (segment (start 231.5 140) (end 247.7 140) (width 1) (layer F.Cu) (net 36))
 (segment (start 204.5125 133.5) (end 204.5 133.4875) (width 0.2) (layer F.Cu) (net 1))
 (segment (start 207.5 133.5) (end 204.5125 133.5) (width 0.2) (layer F.Cu) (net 1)))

